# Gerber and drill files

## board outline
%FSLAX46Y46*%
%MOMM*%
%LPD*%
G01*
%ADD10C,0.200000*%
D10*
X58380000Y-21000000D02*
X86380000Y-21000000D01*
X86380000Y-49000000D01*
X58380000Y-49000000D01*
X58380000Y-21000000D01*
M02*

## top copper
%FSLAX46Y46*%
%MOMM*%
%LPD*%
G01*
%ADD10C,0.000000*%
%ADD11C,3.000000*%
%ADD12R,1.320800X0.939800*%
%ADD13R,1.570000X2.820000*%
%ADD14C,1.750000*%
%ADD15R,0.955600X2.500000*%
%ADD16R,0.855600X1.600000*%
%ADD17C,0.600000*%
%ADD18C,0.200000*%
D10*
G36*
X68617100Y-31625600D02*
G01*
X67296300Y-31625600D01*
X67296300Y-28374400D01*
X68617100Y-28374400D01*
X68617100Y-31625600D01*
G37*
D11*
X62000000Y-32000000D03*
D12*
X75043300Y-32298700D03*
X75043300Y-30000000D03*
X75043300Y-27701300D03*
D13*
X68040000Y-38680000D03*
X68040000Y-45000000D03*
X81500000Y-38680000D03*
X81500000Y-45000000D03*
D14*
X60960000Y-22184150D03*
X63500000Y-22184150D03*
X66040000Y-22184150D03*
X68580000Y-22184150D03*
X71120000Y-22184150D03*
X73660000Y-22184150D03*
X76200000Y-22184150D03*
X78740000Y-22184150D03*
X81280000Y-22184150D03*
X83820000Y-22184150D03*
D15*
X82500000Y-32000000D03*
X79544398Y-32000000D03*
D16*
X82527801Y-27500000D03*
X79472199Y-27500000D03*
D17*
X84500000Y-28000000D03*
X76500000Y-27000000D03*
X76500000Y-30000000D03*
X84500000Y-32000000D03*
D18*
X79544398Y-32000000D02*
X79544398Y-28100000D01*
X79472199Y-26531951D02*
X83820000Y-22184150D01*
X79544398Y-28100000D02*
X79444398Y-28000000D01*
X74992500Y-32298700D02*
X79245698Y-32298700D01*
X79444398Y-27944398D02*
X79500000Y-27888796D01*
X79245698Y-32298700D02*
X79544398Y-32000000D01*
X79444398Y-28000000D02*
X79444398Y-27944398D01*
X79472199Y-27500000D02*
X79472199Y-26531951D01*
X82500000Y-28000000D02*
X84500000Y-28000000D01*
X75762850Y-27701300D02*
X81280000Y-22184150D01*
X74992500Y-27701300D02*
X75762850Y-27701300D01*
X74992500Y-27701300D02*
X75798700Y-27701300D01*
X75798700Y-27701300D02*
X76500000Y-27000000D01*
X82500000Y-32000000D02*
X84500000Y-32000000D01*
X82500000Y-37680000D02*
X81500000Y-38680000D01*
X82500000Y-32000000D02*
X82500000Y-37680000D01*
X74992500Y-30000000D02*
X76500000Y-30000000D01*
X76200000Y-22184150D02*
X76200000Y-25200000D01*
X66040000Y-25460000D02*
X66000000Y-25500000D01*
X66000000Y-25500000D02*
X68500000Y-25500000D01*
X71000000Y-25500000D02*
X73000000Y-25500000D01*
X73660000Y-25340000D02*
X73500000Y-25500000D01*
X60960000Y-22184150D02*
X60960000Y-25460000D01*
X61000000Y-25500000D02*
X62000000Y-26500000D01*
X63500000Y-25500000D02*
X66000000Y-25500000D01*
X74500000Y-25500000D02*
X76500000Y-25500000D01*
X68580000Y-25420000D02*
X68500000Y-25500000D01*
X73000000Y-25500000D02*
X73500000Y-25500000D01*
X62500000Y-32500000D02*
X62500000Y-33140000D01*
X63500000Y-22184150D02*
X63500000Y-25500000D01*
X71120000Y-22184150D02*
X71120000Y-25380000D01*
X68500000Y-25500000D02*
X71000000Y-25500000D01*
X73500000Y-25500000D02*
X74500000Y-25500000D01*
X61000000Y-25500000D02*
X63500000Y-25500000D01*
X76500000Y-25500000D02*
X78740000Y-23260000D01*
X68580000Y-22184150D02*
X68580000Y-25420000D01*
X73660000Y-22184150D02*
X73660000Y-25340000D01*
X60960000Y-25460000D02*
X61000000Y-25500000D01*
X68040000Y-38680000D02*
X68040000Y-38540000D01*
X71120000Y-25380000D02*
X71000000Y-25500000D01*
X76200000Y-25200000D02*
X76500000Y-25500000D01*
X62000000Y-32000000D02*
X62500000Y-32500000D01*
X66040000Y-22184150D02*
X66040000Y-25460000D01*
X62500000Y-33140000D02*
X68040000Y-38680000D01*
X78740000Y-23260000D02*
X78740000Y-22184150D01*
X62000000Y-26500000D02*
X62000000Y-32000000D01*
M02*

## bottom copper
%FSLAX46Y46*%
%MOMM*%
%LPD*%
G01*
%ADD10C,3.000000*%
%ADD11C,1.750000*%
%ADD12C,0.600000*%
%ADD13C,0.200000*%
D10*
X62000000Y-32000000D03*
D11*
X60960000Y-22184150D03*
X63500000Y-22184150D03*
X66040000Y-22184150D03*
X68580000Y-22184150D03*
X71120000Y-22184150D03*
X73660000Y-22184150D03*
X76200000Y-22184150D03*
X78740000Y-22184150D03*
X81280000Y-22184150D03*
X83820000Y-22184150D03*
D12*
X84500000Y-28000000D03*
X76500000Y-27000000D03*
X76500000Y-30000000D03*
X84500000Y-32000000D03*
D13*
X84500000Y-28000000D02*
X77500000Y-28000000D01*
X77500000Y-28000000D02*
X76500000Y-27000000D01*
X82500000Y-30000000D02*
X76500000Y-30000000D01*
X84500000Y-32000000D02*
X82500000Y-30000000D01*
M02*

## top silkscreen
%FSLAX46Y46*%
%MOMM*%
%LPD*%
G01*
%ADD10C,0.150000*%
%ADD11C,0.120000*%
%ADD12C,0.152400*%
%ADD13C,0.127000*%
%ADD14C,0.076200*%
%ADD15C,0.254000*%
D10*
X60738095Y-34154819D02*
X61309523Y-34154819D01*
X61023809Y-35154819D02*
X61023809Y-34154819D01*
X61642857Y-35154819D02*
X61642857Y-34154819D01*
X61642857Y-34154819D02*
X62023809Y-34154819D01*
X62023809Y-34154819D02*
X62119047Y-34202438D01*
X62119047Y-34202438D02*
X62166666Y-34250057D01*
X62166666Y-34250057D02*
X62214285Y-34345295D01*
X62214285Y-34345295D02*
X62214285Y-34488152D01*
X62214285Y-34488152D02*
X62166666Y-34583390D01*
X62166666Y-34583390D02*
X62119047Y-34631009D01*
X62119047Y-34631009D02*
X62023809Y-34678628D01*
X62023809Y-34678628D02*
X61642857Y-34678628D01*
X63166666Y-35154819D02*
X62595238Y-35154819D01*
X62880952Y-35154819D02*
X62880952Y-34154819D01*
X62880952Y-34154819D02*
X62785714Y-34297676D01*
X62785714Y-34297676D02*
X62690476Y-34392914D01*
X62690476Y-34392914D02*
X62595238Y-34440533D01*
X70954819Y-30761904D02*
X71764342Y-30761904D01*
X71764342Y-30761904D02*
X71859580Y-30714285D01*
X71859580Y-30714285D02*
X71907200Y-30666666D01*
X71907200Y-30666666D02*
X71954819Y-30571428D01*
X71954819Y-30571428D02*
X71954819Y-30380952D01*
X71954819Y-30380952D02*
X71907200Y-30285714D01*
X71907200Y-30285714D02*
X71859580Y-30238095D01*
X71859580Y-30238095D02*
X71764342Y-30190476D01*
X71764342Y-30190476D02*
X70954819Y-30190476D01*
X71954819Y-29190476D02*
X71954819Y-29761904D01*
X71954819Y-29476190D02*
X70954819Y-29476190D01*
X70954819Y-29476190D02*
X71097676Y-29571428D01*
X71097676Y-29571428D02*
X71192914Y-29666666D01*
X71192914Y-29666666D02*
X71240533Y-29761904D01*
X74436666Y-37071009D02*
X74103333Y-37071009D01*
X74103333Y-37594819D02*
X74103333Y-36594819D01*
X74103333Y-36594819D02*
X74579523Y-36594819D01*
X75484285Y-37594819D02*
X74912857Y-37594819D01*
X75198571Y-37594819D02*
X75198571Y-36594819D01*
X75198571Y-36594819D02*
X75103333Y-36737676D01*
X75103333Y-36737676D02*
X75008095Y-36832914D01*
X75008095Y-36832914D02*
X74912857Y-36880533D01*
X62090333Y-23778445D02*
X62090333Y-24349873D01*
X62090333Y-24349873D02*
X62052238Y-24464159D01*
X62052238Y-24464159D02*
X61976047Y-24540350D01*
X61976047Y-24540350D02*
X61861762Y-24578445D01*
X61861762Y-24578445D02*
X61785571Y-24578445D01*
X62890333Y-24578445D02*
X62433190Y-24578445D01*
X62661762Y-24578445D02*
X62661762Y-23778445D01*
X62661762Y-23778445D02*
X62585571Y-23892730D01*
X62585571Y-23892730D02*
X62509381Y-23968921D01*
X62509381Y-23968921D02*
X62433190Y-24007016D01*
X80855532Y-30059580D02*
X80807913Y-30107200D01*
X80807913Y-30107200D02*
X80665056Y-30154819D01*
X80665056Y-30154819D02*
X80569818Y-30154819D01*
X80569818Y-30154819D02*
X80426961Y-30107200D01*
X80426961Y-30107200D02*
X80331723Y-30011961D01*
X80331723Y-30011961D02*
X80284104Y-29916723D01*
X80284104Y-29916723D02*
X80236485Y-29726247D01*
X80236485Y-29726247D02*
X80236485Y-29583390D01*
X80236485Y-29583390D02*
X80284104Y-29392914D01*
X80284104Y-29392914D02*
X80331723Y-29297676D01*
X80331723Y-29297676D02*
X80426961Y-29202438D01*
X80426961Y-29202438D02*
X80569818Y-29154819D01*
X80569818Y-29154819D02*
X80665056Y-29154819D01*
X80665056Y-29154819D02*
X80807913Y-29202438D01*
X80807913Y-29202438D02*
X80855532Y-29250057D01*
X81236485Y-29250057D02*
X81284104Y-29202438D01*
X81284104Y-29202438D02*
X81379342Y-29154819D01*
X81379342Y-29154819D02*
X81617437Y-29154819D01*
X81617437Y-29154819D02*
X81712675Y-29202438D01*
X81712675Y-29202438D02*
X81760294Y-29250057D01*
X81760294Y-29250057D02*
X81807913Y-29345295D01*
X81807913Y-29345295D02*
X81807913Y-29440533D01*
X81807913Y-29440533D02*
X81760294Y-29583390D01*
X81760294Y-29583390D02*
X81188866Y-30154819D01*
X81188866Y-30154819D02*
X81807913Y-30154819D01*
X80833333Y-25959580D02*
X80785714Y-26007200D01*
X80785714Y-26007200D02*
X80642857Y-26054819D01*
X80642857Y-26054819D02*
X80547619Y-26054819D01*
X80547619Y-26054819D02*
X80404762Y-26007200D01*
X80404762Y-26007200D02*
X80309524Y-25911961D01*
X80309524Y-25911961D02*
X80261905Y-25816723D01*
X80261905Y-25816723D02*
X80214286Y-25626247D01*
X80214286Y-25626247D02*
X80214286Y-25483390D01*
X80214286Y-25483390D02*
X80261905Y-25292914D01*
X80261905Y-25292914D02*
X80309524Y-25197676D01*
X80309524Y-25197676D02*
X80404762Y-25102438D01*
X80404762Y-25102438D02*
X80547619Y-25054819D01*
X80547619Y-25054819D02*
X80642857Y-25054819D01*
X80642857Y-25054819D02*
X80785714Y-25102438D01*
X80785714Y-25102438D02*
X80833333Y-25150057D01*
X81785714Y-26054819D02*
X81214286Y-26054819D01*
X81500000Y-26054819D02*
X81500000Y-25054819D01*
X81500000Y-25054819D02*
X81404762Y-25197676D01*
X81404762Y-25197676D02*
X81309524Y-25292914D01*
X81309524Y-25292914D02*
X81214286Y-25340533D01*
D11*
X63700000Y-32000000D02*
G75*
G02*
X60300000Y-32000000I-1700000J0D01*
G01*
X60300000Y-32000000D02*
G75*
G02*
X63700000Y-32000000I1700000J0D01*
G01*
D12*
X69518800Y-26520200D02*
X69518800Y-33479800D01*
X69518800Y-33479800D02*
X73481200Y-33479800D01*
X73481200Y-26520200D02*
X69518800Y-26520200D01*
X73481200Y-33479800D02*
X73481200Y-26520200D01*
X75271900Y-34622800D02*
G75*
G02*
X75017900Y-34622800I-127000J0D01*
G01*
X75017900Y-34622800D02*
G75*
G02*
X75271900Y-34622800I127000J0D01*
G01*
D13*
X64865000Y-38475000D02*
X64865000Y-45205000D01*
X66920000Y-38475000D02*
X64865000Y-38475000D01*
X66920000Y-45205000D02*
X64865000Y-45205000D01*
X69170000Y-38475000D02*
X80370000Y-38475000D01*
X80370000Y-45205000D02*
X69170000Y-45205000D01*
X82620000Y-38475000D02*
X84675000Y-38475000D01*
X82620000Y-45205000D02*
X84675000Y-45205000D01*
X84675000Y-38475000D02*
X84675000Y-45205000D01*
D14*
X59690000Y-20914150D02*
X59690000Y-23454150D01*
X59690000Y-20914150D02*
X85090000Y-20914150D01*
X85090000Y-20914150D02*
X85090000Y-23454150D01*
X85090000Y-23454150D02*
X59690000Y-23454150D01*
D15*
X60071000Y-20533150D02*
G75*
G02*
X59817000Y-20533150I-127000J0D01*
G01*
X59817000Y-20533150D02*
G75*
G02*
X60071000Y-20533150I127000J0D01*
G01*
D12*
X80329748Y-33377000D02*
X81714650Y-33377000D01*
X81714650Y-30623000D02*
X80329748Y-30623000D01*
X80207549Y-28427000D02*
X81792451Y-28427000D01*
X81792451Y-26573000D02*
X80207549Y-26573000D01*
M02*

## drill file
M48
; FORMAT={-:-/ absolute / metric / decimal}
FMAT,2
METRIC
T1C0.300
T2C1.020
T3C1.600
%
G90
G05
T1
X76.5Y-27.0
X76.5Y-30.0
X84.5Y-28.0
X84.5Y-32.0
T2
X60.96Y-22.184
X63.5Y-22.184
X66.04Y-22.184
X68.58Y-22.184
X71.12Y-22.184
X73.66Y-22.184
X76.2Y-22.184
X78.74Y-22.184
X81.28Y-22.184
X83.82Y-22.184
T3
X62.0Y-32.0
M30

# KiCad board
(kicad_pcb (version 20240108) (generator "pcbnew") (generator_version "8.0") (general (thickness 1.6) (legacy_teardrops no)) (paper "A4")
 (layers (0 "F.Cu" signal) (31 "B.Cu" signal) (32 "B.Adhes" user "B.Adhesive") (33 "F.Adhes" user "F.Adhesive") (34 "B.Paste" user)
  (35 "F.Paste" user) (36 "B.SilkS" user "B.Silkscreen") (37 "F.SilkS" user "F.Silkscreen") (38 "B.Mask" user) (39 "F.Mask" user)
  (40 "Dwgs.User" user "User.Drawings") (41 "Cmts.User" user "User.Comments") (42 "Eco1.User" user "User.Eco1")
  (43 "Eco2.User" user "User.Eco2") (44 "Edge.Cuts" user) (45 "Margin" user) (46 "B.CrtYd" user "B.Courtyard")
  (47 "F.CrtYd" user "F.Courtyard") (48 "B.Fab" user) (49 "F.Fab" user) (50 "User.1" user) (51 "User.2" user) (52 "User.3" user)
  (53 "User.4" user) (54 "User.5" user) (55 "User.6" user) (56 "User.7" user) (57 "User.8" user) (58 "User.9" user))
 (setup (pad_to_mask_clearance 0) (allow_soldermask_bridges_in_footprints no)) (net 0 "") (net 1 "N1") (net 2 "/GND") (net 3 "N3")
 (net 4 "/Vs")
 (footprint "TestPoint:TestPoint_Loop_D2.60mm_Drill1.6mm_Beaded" (layer "F.Cu") (at 62 32)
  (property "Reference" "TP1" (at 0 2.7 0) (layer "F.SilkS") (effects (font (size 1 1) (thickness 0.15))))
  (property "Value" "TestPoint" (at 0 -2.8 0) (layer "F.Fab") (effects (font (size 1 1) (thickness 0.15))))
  (fp_circle (center 0 0) (end 1.7 0) (stroke (width 0.12) (type solid)) (fill none) (layer "F.SilkS"))
  (pad "1" thru_hole circle (at 0 0) (size 3 3) (drill 1.6) (layers "*.Cu" "*.Mask") (remove_unused_layers no) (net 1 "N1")))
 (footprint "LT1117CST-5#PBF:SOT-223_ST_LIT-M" (layer "F.Cu") (at 71.5 30 90)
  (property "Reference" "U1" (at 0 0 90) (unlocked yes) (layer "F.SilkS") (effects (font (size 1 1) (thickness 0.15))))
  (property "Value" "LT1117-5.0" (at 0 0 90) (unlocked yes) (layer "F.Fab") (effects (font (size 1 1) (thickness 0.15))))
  (fp_poly
   (pts (xy 1.6256 -4.2037) (xy -1.6256 -4.2037) (xy -1.6256 -2.8829) (xy 1.6256 -2.8829)) (stroke (width 0) (type solid)) (fill solid)
   (layer "F.Cu"))
  (fp_line (start 3.4798 -1.9812) (end -3.4798 -1.9812) (stroke (width 0.1524) (type solid)) (layer "F.SilkS"))
  (fp_line (start -3.4798 -1.9812) (end -3.4798 1.9812) (stroke (width 0.1524) (type solid)) (layer "F.SilkS"))
  (fp_line (start 3.4798 1.9812) (end 3.4798 -1.9812) (stroke (width 0.1524) (type solid)) (layer "F.SilkS"))
  (fp_line (start -3.4798 1.9812) (end 3.4798 1.9812) (stroke (width 0.1524) (type solid)) (layer "F.SilkS"))
  (fp_circle (center -4.6228 3.6449) (end -4.4958 3.6449) (stroke (width 0.1524) (type solid)) (fill none) (layer "F.SilkS"))
  (pad "1" smd rect (at -2.2987 3.5433 90) (size 0.9398 1.3208) (layers "F.Cu" "F.Paste" "F.Mask") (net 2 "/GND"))
  (pad "2" smd rect (at 0 3.5433 90) (size 0.9398 1.3208) (layers "F.Cu" "F.Paste" "F.Mask") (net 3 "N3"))
  (pad "3" smd rect (at 2.2987 3.5433 90) (size 0.9398 1.3208) (layers "F.Cu" "F.Paste" "F.Mask") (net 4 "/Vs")))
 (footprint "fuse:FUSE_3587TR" (layer "F.Cu") (at 74.77 41.84)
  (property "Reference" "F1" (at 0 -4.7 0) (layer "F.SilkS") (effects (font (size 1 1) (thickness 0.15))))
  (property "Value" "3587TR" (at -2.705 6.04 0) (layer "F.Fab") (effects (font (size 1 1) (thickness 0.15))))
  (fp_line (start -9.905 -3.365) (end -9.905 3.365) (stroke (width 0.127) (type solid)) (layer "F.SilkS"))
  (fp_line (start -7.85 -3.365) (end -9.905 -3.365) (stroke (width 0.127) (type solid)) (layer "F.SilkS"))
  (fp_line (start -7.85 3.365) (end -9.905 3.365) (stroke (width 0.127) (type solid)) (layer "F.SilkS"))
  (fp_line (start -5.6 -3.365) (end 5.6 -3.365) (stroke (width 0.127) (type solid)) (layer "F.SilkS"))
  (fp_line (start 5.6 3.365) (end -5.6 3.365) (stroke (width 0.127) (type solid)) (layer "F.SilkS"))
  (fp_line (start 7.85 -3.365) (end 9.905 -3.365) (stroke (width 0.127) (type solid)) (layer "F.SilkS"))
  (fp_line (start 7.85 3.365) (end 9.905 3.365) (stroke (width 0.127) (type solid)) (layer "F.SilkS"))
  (fp_line (start 9.905 -3.365) (end 9.905 3.365) (stroke (width 0.127) (type solid)) (layer "F.SilkS"))
  (pad "1_1" smd rect (at -6.73 -3.16) (size 1.57 2.82) (layers "F.Cu" "F.Paste" "F.Mask") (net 1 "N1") (solder_mask_margin 0.102))
  (pad "1_2" smd rect (at -6.73 3.16) (size 1.57 2.82) (layers "F.Cu" "F.Paste" "F.Mask") (solder_mask_margin 0.102))
  (pad "2_1" smd rect (at 6.73 -3.16) (size 1.57 2.82) (layers "F.Cu" "F.Paste" "F.Mask") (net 3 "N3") (solder_mask_margin 0.102))
  (pad "2_2" smd rect (at 6.73 3.16) (size 1.57 2.82) (layers "F.Cu" "F.Paste" "F.Mask") (solder_mask_margin 0.102)))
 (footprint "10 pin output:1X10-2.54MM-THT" (layer "F.Cu") (at 60.96 22.18415)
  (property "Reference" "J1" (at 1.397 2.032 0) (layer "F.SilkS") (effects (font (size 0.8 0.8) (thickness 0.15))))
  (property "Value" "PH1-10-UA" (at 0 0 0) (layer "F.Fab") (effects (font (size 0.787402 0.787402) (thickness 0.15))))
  (fp_line (start -1.27 -1.27) (end -1.27 1.27) (stroke (width 0.0762) (type solid)) (layer "F.SilkS"))
  (fp_line (start -1.27 -1.27) (end 24.13 -1.27) (stroke (width 0.0762) (type solid)) (layer "F.SilkS"))
  (fp_line (start 24.13 -1.27) (end 24.13 1.27) (stroke (width 0.0762) (type solid)) (layer "F.SilkS"))
  (fp_line (start 24.13 1.27) (end -1.27 1.27) (stroke (width 0.0762) (type solid)) (layer "F.SilkS"))
  (fp_circle (center -1.016 -1.651) (end -0.762 -1.651) (stroke (width 0) (type solid)) (fill solid) (layer "F.SilkS"))
  (pad "1" thru_hole circle (at 0 0) (size 1.75 1.75) (drill 1.02) (layers "*.Cu" "*.Mask") (remove_unused_layers no) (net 1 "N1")
   (solder_mask_margin 0.102))
  (pad "2" thru_hole circle (at 2.54 0) (size 1.75 1.75) (drill 1.02) (layers "*.Cu" "*.Mask") (remove_unused_layers no) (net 1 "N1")
   (solder_mask_margin 0.102))
  (pad "3" thru_hole circle (at 5.08 0) (size 1.75 1.75) (drill 1.02) (layers "*.Cu" "*.Mask") (remove_unused_layers no) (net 1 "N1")
   (solder_mask_margin 0.102))
  (pad "4" thru_hole circle (at 7.62 0) (size 1.75 1.75) (drill 1.02) (layers "*.Cu" "*.Mask") (remove_unused_layers no) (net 1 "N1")
   (solder_mask_margin 0.102))
  (pad "5" thru_hole circle (at 10.16 0) (size 1.75 1.75) (drill 1.02) (layers "*.Cu" "*.Mask") (remove_unused_layers no) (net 1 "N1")
   (solder_mask_margin 0.102))
  (pad "6" thru_hole circle (at 12.7 0) (size 1.75 1.75) (drill 1.02) (layers "*.Cu" "*.Mask") (remove_unused_layers no) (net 1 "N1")
   (solder_mask_margin 0.102))
  (pad "7" thru_hole circle (at 15.24 0) (size 1.75 1.75) (drill 1.02) (layers "*.Cu" "*.Mask") (remove_unused_layers no) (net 1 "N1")
   (solder_mask_margin 0.102))
  (pad "8" thru_hole circle (at 17.78 0) (size 1.75 1.75) (drill 1.02) (layers "*.Cu" "*.Mask") (remove_unused_layers no) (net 1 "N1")
   (solder_mask_margin 0.102))
  (pad "9" thru_hole circle (at 20.32 0) (size 1.75 1.75) (drill 1.02) (layers "*.Cu" "*.Mask") (remove_unused_layers no) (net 4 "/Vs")
   (solder_mask_margin 0.102))
  (pad "10" thru_hole circle (at 22.86 0) (size 1.75 1.75) (drill 1.02) (layers "*.Cu" "*.Mask") (remove_unused_layers no) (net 2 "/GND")
   (solder_mask_margin 0.102)))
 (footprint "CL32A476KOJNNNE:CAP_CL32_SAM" (layer "F.Cu") (at 81.022199 32 180)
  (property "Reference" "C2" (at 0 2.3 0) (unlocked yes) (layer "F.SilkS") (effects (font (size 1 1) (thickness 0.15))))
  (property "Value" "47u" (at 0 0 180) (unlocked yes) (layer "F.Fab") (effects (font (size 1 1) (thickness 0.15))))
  (fp_line (start 0.692451 -1.377) (end -0.692451 -1.377) (stroke (width 0.1524) (type solid)) (layer "F.SilkS"))
  (fp_line (start -0.692451 1.377) (end 0.692451 1.377) (stroke (width 0.1524) (type solid)) (layer "F.SilkS"))
  (pad "1" smd rect (at -1.477801 0 180) (size 0.9556 2.5) (layers "F.Cu" "F.Paste" "F.Mask") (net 3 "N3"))
  (pad "2" smd rect (at 1.477801 0 180) (size 0.9556 2.5) (layers "F.Cu" "F.Paste" "F.Mask") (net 2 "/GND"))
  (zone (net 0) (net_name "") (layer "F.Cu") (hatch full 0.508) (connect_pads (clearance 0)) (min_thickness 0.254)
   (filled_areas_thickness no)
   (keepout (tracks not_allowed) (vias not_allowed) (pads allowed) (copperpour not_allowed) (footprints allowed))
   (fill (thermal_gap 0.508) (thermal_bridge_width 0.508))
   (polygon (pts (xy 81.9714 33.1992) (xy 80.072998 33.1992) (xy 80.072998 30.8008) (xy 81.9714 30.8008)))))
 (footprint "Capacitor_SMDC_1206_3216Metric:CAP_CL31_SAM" (layer "F.Cu") (at 81 27.5 180)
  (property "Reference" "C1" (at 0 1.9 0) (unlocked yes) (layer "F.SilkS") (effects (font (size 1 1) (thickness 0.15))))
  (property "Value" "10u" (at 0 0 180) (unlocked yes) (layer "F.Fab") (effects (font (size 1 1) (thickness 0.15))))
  (fp_line (start 0.792451 -0.927) (end -0.792451 -0.927) (stroke (width 0.1524) (type solid)) (layer "F.SilkS"))
  (fp_line (start -0.792451 0.927) (end 0.792451 0.927) (stroke (width 0.1524) (type solid)) (layer "F.SilkS"))
  (pad "1" smd rect (at -1.527801 0 180) (size 0.8556 1.6) (layers "F.Cu" "F.Paste" "F.Mask") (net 4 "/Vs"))
  (pad "2" smd rect (at 1.527801 0 180) (size 0.8556 1.6) (layers "F.Cu" "F.Paste" "F.Mask") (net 2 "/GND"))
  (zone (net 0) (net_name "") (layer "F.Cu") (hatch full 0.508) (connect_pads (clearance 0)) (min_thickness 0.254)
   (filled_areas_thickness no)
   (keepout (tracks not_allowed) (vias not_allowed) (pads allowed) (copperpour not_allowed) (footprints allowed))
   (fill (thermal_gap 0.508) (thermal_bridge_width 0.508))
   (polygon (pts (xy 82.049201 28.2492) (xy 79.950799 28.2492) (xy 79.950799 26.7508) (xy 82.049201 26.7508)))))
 (gr_rect (start 58.38 21) (end 86.38 49) (stroke (width 0.2) (type default)) (fill none) (layer "Edge.Cuts"))
 (segment (start 79.544398 32) (end 79.544398 28.1) (width 0.2) (layer "F.Cu") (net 2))
 (segment (start 79.472199 26.531951) (end 83.82 22.18415) (width 0.2) (layer "F.Cu") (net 2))
 (segment (start 79.544398 28.1) (end 79.444398 28) (width 0.2) (layer "F.Cu") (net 2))
 (segment (start 74.9925 32.2987) (end 79.245698 32.2987) (width 0.2) (layer "F.Cu") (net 2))
 (segment (start 79.444398 27.944398) (end 79.5 27.888796) (width 0.2) (layer "F.Cu") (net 2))
 (segment (start 79.245698 32.2987) (end 79.544398 32) (width 0.2) (layer "F.Cu") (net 2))
 (segment (start 79.444398 28) (end 79.444398 27.944398) (width 0.2) (layer "F.Cu") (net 2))
 (segment (start 79.472199 27.5) (end 79.472199 26.531951) (width 0.2) (layer "F.Cu") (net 2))
 (segment (start 82.5 28) (end 84.5 28) (width 0.2) (layer "F.Cu") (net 4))
 (segment (start 75.76285 27.7013) (end 81.28 22.18415) (width 0.2) (layer "F.Cu") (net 4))
 (segment (start 74.9925 27.7013) (end 75.76285 27.7013) (width 0.2) (layer "F.Cu") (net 4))
 (segment (start 74.9925 27.7013) (end 75.7987 27.7013) (width 0.2) (layer "F.Cu") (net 4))
 (segment (start 75.7987 27.7013) (end 76.5 27) (width 0.2) (layer "F.Cu") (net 4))
 (via (at 84.5 28) (size 0.6) (drill 0.3) (layers "F.Cu" "B.Cu") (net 4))
 (via (at 76.5 27) (size 0.6) (drill 0.3) (layers "F.Cu" "B.Cu") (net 4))
 (segment (start 84.5 28) (end 77.5 28) (width 0.2) (layer "B.Cu") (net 4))
 (segment (start 77.5 28) (end 76.5 27) (width 0.2) (layer "B.Cu") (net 4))
 (segment (start 82.5 32) (end 84.5 32) (width 0.2) (layer "F.Cu") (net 3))
 (segment (start 82.5 37.68) (end 81.5 38.68) (width 0.2) (layer "F.Cu") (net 3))
 (segment (start 82.5 32) (end 82.5 37.68) (width 0.2) (layer "F.Cu") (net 3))
 (segment (start 74.9925 30) (end 76.5 30) (width 0.2) (layer "F.Cu") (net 3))
 (via (at 76.5 30) (size 0.6) (drill 0.3) (layers "F.Cu" "B.Cu") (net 3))
 (via (at 84.5 32) (size 0.6) (drill 0.3) (layers "F.Cu" "B.Cu") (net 3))
 (segment (start 82.5 30) (end 76.5 30) (width 0.2) (layer "B.Cu") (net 3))
 (segment (start 84.5 32) (end 82.5 30) (width 0.2) (layer "B.Cu") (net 3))
 (segment (start 76.2 22.18415) (end 76.2 25.2) (width 0.2) (layer "F.Cu") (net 1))
 (segment (start 66.04 25.46) (end 66 25.5) (width 0.2) (layer "F.Cu") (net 1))
 (segment (start 66 25.5) (end 68.5 25.5) (width 0.2) (layer "F.Cu") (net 1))
 (segment (start 71 25.5) (end 73 25.5) (width 0.2) (layer "F.Cu") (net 1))
 (segment (start 73.66 25.34) (end 73.5 25.5) (width 0.2) (layer "F.Cu") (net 1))
 (segment (start 60.96 22.18415) (end 60.96 25.46) (width 0.2) (layer "F.Cu") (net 1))
 (segment (start 61 25.5) (end 62 26.5) (width 0.2) (layer "F.Cu") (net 1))
 (segment (start 63.5 25.5) (end 66 25.5) (width 0.2) (layer "F.Cu") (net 1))
 (segment (start 74.5 25.5) (end 76.5 25.5) (width 0.2) (layer "F.Cu") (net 1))
 (segment (start 68.58 25.42) (end 68.5 25.5) (width 0.2) (layer "F.Cu") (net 1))
 (segment (start 73 25.5) (end 73.5 25.5) (width 0.2) (layer "F.Cu") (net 1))
 (segment (start 62.5 32.5) (end 62.5 33.14) (width 0.2) (layer "F.Cu") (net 1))
 (segment (start 63.5 22.18415) (end 63.5 25.5) (width 0.2) (layer "F.Cu") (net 1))
 (segment (start 71.12 22.18415) (end 71.12 25.38) (width 0.2) (layer "F.Cu") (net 1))
 (segment (start 68.5 25.5) (end 71 25.5) (width 0.2) (layer "F.Cu") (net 1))
 (segment (start 73.5 25.5) (end 74.5 25.5) (width 0.2) (layer "F.Cu") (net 1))
 (segment (start 61 25.5) (end 63.5 25.5) (width 0.2) (layer "F.Cu") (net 1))
 (segment (start 76.5 25.5) (end 78.74 23.26) (width 0.2) (layer "F.Cu") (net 1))
 (segment (start 68.58 22.18415) (end 68.58 25.42) (width 0.2) (layer "F.Cu") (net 1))
 (segment (start 73.66 22.18415) (end 73.66 25.34) (width 0.2) (layer "F.Cu") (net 1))
 (segment (start 60.96 25.46) (end 61 25.5) (width 0.2) (layer "F.Cu") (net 1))
 (segment (start 68.04 38.68) (end 68.04 38.54) (width 0.2) (layer "F.Cu") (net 1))
 (segment (start 71.12 25.38) (end 71 25.5) (width 0.2) (layer "F.Cu") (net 1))
 (segment (start 76.2 25.2) (end 76.5 25.5) (width 0.2) (layer "F.Cu") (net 1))
 (segment (start 62 32) (end 62.5 32.5) (width 0.2) (layer "F.Cu") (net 1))
 (segment (start 66.04 22.18415) (end 66.04 25.46) (width 0.2) (layer "F.Cu") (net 1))
 (segment (start 62.5 33.14) (end 68.04 38.68) (width 0.2) (layer "F.Cu") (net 1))
 (segment (start 78.74 23.26) (end 78.74 22.18415) (width 0.2) (layer "F.Cu") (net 1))
 (segment (start 62 26.5) (end 62 32) (width 0.2) (layer "F.Cu") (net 1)))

